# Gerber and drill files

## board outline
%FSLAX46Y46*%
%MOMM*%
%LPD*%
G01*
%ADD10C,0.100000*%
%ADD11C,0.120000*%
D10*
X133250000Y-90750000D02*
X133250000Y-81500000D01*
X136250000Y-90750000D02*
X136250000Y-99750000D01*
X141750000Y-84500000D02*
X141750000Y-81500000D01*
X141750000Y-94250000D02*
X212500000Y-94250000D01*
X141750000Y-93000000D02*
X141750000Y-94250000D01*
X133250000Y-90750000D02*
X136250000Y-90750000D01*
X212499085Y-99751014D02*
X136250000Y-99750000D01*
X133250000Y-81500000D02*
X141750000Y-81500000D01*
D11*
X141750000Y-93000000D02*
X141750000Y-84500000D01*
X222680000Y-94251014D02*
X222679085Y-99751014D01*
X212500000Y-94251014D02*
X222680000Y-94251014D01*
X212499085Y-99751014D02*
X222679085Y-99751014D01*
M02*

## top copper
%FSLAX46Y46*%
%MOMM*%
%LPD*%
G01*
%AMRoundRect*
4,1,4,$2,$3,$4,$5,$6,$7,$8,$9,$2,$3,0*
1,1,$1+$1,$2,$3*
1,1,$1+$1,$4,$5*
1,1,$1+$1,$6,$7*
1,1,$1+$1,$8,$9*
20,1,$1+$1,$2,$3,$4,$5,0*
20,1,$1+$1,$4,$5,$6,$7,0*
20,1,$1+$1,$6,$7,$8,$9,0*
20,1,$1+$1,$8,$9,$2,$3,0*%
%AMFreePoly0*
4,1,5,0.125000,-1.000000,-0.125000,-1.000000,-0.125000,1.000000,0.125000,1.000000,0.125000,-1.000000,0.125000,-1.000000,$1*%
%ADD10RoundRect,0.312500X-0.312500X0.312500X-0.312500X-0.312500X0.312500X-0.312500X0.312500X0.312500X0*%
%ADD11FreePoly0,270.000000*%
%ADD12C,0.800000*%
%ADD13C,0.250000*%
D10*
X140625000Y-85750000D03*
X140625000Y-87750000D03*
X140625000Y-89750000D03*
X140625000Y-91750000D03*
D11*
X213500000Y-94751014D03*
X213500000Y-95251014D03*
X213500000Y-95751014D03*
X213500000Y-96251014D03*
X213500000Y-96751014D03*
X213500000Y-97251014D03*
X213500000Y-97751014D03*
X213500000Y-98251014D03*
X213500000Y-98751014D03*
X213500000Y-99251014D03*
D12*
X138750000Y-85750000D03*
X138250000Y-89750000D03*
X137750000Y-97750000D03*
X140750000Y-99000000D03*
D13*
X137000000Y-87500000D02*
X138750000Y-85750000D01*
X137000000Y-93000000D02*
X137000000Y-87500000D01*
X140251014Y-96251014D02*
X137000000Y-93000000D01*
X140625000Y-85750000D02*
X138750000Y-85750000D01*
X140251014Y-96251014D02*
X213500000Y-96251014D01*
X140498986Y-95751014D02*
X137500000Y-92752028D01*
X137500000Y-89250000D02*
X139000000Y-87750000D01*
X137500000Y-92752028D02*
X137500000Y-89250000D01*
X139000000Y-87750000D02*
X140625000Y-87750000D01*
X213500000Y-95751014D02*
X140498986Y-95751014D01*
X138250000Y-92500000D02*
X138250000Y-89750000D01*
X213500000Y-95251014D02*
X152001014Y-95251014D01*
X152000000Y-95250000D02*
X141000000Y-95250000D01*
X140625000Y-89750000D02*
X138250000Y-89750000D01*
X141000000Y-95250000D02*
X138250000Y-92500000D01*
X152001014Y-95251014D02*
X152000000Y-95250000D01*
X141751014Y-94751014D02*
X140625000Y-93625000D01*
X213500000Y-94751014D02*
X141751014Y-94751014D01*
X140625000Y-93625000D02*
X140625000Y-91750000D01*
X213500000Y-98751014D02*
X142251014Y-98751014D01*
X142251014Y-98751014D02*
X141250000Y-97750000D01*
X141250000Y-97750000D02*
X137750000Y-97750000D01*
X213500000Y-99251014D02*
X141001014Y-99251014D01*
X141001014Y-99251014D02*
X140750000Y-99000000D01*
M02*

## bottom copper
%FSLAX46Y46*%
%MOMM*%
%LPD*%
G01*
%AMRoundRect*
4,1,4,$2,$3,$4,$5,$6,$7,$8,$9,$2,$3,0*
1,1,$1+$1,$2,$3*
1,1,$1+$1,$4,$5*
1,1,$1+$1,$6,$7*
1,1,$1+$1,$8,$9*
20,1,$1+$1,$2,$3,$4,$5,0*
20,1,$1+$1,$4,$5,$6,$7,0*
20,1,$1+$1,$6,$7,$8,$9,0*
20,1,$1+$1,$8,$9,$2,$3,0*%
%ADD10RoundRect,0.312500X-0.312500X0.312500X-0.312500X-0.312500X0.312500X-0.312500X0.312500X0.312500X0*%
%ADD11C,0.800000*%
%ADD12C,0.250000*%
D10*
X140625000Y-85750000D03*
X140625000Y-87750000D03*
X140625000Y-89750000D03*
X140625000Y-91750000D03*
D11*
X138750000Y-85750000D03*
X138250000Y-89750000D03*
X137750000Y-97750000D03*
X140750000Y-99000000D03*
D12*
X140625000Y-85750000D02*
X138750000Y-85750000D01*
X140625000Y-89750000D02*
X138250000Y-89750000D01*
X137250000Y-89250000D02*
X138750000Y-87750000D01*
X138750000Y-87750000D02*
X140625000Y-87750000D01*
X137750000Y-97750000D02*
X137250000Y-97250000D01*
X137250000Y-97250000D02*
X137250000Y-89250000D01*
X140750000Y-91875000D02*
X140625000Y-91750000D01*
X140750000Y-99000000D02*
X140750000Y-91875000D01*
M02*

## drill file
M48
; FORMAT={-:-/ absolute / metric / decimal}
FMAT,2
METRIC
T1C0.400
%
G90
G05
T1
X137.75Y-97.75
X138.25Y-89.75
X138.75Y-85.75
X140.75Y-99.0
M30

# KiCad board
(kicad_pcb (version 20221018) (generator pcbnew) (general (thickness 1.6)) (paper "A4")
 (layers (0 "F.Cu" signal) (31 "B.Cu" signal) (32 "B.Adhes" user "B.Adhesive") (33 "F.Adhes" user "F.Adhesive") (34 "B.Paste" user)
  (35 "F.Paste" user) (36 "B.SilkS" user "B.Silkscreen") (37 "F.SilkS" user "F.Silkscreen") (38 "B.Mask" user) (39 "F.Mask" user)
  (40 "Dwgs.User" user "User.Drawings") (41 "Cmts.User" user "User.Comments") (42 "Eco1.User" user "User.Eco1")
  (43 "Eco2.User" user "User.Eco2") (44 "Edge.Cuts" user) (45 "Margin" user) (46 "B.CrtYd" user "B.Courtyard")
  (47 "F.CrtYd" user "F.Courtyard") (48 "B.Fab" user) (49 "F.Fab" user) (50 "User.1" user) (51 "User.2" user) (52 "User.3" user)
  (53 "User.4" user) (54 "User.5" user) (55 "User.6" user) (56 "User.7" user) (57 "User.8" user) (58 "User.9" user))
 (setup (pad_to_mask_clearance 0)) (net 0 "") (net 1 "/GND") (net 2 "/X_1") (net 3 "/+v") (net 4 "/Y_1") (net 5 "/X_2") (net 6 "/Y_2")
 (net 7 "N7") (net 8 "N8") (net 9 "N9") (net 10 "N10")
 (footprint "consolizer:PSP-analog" (layer "F.Cu") (at 140.75 88 -90)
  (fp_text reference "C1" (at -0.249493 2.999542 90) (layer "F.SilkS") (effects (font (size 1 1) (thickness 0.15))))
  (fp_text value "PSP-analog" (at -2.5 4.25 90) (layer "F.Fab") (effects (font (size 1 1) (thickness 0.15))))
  (fp_line (start 5 -1) (end -3.5 -1) (stroke (width 0.12) (type solid)) (layer "Edge.Cuts"))
  (pad "1" smd roundrect (at -2.25 0.125 270) (size 1.25 1.25) (layers "F.Cu" "F.Paste" "F.Mask") (roundrect_rratio 0.25) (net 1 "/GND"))
  (pad "2" smd roundrect (at -0.25 0.125 270) (size 1.25 1.25) (layers "F.Cu" "F.Paste" "F.Mask") (roundrect_rratio 0.25) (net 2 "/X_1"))
  (pad "3" smd roundrect (at 1.75 0.125 270) (size 1.25 1.25) (layers "F.Cu" "F.Paste" "F.Mask") (roundrect_rratio 0.25) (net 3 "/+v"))
  (pad "4" smd roundrect (at 3.75 0.125 270) (size 1.25 1.25) (layers "F.Cu" "F.Paste" "F.Mask") (roundrect_rratio 0.25) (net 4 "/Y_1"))
  (pad "5" smd roundrect (at -2.25 0.125 270) (size 1.25 1.25) (layers "B.Cu" "B.Paste" "B.Mask") (roundrect_rratio 0.25) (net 1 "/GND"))
  (pad "6" smd roundrect (at -0.25 0.125 270) (size 1.25 1.25) (layers "B.Cu" "B.Paste" "B.Mask") (roundrect_rratio 0.25) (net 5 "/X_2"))
  (pad "7" smd roundrect (at 1.75 0.125 270) (size 1.25 1.25) (layers "B.Cu" "B.Paste" "B.Mask") (roundrect_rratio 0.25) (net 3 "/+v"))
  (pad "8" smd roundrect (at 3.75 0.125 270) (size 1.25 1.25) (layers "B.Cu" "B.Paste" "B.Mask") (roundrect_rratio 0.25) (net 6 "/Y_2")))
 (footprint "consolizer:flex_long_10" (layer "F.Cu") (at 218.5 97.251014 -90)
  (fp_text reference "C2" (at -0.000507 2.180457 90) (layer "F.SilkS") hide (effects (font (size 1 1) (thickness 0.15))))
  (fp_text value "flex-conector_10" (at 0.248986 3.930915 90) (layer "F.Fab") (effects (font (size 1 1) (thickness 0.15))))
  (fp_line (start -3 -4.18) (end 2.5 -4.179085) (stroke (width 0.12) (type solid)) (layer "Edge.Cuts"))
  (fp_line (start -3 6) (end -3 -4.18) (stroke (width 0.12) (type solid)) (layer "Edge.Cuts"))
  (fp_line (start 2.5 6.000915) (end 2.5 -4.179085) (stroke (width 0.12) (type solid)) (layer "Edge.Cuts"))
  (pad "" smd rect (at -2.5 -2 270) (size 0.25 4) (layers "F.Paste" "F.Mask"))
  (pad "" smd rect (at -2 -2 270) (size 0.25 4) (layers "F.Paste" "F.Mask"))
  (pad "" smd rect (at -1.5 -2 270) (size 0.25 4) (layers "F.Paste" "F.Mask"))
  (pad "" smd rect (at -1 -2 270) (size 0.25 4) (layers "F.Paste" "F.Mask"))
  (pad "" smd rect (at -0.5 -2 270) (size 0.25 4) (layers "F.Paste" "F.Mask"))
  (pad "" smd rect (at 0 -2 270) (size 0.25 4) (layers "F.Paste" "F.Mask"))
  (pad "" smd rect (at 0.5 -2 270) (size 0.25 4) (layers "F.Paste" "F.Mask"))
  (pad "" smd rect (at 1 -2 270) (size 0.25 4) (layers "F.Paste" "F.Mask"))
  (pad "" smd rect (at 1.5 -2 270) (size 0.25 4) (layers "F.Paste" "F.Mask"))
  (pad "" smd rect (at 1.998986 -1.999085 270) (size 0.25 4) (layers "F.Paste" "F.Mask"))
  (pad "1" smd custom (at -2.5 5 270) (size 0.25 2) (layers "F.Cu") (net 4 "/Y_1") (zone_connect 0) (thermal_bridge_angle 45)
   (options (clearance outline) (anchor rect)) (primitives))
  (pad "2" smd custom (at -2 5 270) (size 0.25 2) (layers "F.Cu") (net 3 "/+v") (zone_connect 0) (thermal_bridge_angle 45)
   (options (clearance outline) (anchor rect)) (primitives))
  (pad "3" smd custom (at -1.5 5 270) (size 0.25 2) (layers "F.Cu") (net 2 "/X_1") (zone_connect 0) (thermal_bridge_angle 45)
   (options (clearance outline) (anchor rect)) (primitives))
  (pad "4" smd custom (at -1 5 270) (size 0.25 2) (layers "F.Cu") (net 1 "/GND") (zone_connect 0) (thermal_bridge_angle 45)
   (options (clearance outline) (anchor rect)) (primitives))
  (pad "5" smd custom (at -0.5 5 270) (size 0.25 2) (layers "F.Cu") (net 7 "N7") (zone_connect 0) (thermal_bridge_angle 45)
   (options (clearance outline) (anchor rect)) (primitives))
  (pad "6" smd custom (at 0 5 270) (size 0.25 2) (layers "F.Cu") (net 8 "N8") (zone_connect 0) (thermal_bridge_angle 45)
   (options (clearance outline) (anchor rect)) (primitives))
  (pad "7" smd custom (at 0.5 5 270) (size 0.25 2) (layers "F.Cu") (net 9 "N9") (zone_connect 0) (thermal_bridge_angle 45)
   (options (clearance outline) (anchor rect)) (primitives))
  (pad "8" smd custom (at 1 5 270) (size 0.25 2) (layers "F.Cu") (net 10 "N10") (zone_connect 0) (thermal_bridge_angle 45)
   (options (clearance outline) (anchor rect)) (primitives))
  (pad "9" smd custom (at 1.5 5 270) (size 0.25 2) (layers "F.Cu") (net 5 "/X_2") (zone_connect 0) (thermal_bridge_angle 45)
   (options (clearance outline) (anchor rect)) (primitives))
  (pad "10" smd custom (at 2 5 270) (size 0.25 2) (layers "F.Cu") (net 6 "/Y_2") (zone_connect 0) (thermal_bridge_angle 45)
   (options (clearance outline) (anchor rect)) (primitives)))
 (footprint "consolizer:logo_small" (layer "F.Cu") (at 192 97)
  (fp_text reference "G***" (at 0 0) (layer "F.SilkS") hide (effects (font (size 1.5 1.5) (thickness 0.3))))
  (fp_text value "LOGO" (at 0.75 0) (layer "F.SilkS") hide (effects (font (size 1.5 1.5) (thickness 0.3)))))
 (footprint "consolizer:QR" (layer "B.Cu") (at 147.25 69 -90)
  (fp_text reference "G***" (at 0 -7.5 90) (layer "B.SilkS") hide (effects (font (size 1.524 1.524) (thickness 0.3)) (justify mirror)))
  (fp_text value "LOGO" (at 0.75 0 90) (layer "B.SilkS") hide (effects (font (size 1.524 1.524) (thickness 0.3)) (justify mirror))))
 (gr_line (start 133.25 90.75) (end 133.25 81.5) (stroke (width 0.1) (type solid)) (layer "Edge.Cuts"))
 (gr_line (start 136.25 90.75) (end 136.25 99.75) (stroke (width 0.1) (type solid)) (layer "Edge.Cuts"))
 (gr_line (start 141.75 84.5) (end 141.75 81.5) (stroke (width 0.1) (type default)) (layer "Edge.Cuts"))
 (gr_line (start 141.75 94.25) (end 212.5 94.25) (stroke (width 0.1) (type default)) (layer "Edge.Cuts"))
 (gr_line (start 141.75 93) (end 141.75 94.25) (stroke (width 0.1) (type default)) (layer "Edge.Cuts"))
 (gr_line (start 133.25 90.75) (end 136.25 90.75) (stroke (width 0.1) (type solid)) (layer "Edge.Cuts"))
 (gr_line (start 212.499085 99.751014) (end 136.25 99.75) (stroke (width 0.1) (type default)) (layer "Edge.Cuts"))
 (gr_line (start 133.25 81.5) (end 141.75 81.5) (stroke (width 0.1) (type solid)) (layer "Edge.Cuts"))
 (segment (start 137 87.5) (end 138.75 85.75) (width 0.25) (layer "F.Cu") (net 1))
 (segment (start 137 93) (end 137 87.5) (width 0.25) (layer "F.Cu") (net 1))
 (segment (start 140.251014 96.251014) (end 137 93) (width 0.25) (layer "F.Cu") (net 1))
 (segment (start 140.625 85.75) (end 138.75 85.75) (width 0.25) (layer "F.Cu") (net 1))
 (segment (start 140.251014 96.251014) (end 213.5 96.251014) (width 0.25) (layer "F.Cu") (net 1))
 (via (at 138.75 85.75) (size 0.8) (drill 0.4) (layers "F.Cu" "B.Cu") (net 1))
 (segment (start 140.625 85.75) (end 138.75 85.75) (width 0.25) (layer "B.Cu") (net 1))
 (segment (start 140.498986 95.751014) (end 137.5 92.752028) (width 0.25) (layer "F.Cu") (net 2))
 (segment (start 137.5 89.25) (end 139 87.75) (width 0.25) (layer "F.Cu") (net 2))
 (segment (start 137.5 92.752028) (end 137.5 89.25) (width 0.25) (layer "F.Cu") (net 2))
 (segment (start 139 87.75) (end 140.625 87.75) (width 0.25) (layer "F.Cu") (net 2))
 (segment (start 213.5 95.751014) (end 140.498986 95.751014) (width 0.25) (layer "F.Cu") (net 2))
 (segment (start 138.25 92.5) (end 138.25 89.75) (width 0.25) (layer "F.Cu") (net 3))
 (segment (start 213.5 95.251014) (end 152.001014 95.251014) (width 0.25) (layer "F.Cu") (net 3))
 (segment (start 152 95.25) (end 141 95.25) (width 0.25) (layer "F.Cu") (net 3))
 (segment (start 140.625 89.75) (end 138.25 89.75) (width 0.25) (layer "F.Cu") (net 3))
 (segment (start 141 95.25) (end 138.25 92.5) (width 0.25) (layer "F.Cu") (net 3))
 (segment (start 152.001014 95.251014) (end 152 95.25) (width 0.25) (layer "F.Cu") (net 3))
 (via (at 138.25 89.75) (size 0.8) (drill 0.4) (layers "F.Cu" "B.Cu") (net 3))
 (segment (start 140.625 89.75) (end 138.25 89.75) (width 0.25) (layer "B.Cu") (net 3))
 (segment (start 141.751014 94.751014) (end 140.625 93.625) (width 0.25) (layer "F.Cu") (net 4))
 (segment (start 213.5 94.751014) (end 141.751014 94.751014) (width 0.25) (layer "F.Cu") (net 4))
 (segment (start 140.625 93.625) (end 140.625 91.75) (width 0.25) (layer "F.Cu") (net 4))
 (segment (start 213.5 98.751014) (end 142.251014 98.751014) (width 0.25) (layer "F.Cu") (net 5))
 (segment (start 142.251014 98.751014) (end 141.25 97.75) (width 0.25) (layer "F.Cu") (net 5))
 (segment (start 141.25 97.75) (end 137.75 97.75) (width 0.25) (layer "F.Cu") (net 5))
 (via (at 137.75 97.75) (size 0.8) (drill 0.4) (layers "F.Cu" "B.Cu") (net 5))
 (segment (start 137.25 89.25) (end 138.75 87.75) (width 0.25) (layer "B.Cu") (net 5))
 (segment (start 138.75 87.75) (end 140.625 87.75) (width 0.25) (layer "B.Cu") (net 5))
 (segment (start 137.75 97.75) (end 137.25 97.25) (width 0.25) (layer "B.Cu") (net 5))
 (segment (start 137.25 97.25) (end 137.25 89.25) (width 0.25) (layer "B.Cu") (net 5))
 (segment (start 213.5 99.251014) (end 141.001014 99.251014) (width 0.25) (layer "F.Cu") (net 6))
 (segment (start 141.001014 99.251014) (end 140.75 99) (width 0.25) (layer "F.Cu") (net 6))
 (via (at 140.75 99) (size 0.8) (drill 0.4) (layers "F.Cu" "B.Cu") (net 6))
 (segment (start 140.75 91.875) (end 140.625 91.75) (width 0.25) (layer "B.Cu") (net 6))
 (segment (start 140.75 99) (end 140.75 91.875) (width 0.25) (layer "B.Cu") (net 6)))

